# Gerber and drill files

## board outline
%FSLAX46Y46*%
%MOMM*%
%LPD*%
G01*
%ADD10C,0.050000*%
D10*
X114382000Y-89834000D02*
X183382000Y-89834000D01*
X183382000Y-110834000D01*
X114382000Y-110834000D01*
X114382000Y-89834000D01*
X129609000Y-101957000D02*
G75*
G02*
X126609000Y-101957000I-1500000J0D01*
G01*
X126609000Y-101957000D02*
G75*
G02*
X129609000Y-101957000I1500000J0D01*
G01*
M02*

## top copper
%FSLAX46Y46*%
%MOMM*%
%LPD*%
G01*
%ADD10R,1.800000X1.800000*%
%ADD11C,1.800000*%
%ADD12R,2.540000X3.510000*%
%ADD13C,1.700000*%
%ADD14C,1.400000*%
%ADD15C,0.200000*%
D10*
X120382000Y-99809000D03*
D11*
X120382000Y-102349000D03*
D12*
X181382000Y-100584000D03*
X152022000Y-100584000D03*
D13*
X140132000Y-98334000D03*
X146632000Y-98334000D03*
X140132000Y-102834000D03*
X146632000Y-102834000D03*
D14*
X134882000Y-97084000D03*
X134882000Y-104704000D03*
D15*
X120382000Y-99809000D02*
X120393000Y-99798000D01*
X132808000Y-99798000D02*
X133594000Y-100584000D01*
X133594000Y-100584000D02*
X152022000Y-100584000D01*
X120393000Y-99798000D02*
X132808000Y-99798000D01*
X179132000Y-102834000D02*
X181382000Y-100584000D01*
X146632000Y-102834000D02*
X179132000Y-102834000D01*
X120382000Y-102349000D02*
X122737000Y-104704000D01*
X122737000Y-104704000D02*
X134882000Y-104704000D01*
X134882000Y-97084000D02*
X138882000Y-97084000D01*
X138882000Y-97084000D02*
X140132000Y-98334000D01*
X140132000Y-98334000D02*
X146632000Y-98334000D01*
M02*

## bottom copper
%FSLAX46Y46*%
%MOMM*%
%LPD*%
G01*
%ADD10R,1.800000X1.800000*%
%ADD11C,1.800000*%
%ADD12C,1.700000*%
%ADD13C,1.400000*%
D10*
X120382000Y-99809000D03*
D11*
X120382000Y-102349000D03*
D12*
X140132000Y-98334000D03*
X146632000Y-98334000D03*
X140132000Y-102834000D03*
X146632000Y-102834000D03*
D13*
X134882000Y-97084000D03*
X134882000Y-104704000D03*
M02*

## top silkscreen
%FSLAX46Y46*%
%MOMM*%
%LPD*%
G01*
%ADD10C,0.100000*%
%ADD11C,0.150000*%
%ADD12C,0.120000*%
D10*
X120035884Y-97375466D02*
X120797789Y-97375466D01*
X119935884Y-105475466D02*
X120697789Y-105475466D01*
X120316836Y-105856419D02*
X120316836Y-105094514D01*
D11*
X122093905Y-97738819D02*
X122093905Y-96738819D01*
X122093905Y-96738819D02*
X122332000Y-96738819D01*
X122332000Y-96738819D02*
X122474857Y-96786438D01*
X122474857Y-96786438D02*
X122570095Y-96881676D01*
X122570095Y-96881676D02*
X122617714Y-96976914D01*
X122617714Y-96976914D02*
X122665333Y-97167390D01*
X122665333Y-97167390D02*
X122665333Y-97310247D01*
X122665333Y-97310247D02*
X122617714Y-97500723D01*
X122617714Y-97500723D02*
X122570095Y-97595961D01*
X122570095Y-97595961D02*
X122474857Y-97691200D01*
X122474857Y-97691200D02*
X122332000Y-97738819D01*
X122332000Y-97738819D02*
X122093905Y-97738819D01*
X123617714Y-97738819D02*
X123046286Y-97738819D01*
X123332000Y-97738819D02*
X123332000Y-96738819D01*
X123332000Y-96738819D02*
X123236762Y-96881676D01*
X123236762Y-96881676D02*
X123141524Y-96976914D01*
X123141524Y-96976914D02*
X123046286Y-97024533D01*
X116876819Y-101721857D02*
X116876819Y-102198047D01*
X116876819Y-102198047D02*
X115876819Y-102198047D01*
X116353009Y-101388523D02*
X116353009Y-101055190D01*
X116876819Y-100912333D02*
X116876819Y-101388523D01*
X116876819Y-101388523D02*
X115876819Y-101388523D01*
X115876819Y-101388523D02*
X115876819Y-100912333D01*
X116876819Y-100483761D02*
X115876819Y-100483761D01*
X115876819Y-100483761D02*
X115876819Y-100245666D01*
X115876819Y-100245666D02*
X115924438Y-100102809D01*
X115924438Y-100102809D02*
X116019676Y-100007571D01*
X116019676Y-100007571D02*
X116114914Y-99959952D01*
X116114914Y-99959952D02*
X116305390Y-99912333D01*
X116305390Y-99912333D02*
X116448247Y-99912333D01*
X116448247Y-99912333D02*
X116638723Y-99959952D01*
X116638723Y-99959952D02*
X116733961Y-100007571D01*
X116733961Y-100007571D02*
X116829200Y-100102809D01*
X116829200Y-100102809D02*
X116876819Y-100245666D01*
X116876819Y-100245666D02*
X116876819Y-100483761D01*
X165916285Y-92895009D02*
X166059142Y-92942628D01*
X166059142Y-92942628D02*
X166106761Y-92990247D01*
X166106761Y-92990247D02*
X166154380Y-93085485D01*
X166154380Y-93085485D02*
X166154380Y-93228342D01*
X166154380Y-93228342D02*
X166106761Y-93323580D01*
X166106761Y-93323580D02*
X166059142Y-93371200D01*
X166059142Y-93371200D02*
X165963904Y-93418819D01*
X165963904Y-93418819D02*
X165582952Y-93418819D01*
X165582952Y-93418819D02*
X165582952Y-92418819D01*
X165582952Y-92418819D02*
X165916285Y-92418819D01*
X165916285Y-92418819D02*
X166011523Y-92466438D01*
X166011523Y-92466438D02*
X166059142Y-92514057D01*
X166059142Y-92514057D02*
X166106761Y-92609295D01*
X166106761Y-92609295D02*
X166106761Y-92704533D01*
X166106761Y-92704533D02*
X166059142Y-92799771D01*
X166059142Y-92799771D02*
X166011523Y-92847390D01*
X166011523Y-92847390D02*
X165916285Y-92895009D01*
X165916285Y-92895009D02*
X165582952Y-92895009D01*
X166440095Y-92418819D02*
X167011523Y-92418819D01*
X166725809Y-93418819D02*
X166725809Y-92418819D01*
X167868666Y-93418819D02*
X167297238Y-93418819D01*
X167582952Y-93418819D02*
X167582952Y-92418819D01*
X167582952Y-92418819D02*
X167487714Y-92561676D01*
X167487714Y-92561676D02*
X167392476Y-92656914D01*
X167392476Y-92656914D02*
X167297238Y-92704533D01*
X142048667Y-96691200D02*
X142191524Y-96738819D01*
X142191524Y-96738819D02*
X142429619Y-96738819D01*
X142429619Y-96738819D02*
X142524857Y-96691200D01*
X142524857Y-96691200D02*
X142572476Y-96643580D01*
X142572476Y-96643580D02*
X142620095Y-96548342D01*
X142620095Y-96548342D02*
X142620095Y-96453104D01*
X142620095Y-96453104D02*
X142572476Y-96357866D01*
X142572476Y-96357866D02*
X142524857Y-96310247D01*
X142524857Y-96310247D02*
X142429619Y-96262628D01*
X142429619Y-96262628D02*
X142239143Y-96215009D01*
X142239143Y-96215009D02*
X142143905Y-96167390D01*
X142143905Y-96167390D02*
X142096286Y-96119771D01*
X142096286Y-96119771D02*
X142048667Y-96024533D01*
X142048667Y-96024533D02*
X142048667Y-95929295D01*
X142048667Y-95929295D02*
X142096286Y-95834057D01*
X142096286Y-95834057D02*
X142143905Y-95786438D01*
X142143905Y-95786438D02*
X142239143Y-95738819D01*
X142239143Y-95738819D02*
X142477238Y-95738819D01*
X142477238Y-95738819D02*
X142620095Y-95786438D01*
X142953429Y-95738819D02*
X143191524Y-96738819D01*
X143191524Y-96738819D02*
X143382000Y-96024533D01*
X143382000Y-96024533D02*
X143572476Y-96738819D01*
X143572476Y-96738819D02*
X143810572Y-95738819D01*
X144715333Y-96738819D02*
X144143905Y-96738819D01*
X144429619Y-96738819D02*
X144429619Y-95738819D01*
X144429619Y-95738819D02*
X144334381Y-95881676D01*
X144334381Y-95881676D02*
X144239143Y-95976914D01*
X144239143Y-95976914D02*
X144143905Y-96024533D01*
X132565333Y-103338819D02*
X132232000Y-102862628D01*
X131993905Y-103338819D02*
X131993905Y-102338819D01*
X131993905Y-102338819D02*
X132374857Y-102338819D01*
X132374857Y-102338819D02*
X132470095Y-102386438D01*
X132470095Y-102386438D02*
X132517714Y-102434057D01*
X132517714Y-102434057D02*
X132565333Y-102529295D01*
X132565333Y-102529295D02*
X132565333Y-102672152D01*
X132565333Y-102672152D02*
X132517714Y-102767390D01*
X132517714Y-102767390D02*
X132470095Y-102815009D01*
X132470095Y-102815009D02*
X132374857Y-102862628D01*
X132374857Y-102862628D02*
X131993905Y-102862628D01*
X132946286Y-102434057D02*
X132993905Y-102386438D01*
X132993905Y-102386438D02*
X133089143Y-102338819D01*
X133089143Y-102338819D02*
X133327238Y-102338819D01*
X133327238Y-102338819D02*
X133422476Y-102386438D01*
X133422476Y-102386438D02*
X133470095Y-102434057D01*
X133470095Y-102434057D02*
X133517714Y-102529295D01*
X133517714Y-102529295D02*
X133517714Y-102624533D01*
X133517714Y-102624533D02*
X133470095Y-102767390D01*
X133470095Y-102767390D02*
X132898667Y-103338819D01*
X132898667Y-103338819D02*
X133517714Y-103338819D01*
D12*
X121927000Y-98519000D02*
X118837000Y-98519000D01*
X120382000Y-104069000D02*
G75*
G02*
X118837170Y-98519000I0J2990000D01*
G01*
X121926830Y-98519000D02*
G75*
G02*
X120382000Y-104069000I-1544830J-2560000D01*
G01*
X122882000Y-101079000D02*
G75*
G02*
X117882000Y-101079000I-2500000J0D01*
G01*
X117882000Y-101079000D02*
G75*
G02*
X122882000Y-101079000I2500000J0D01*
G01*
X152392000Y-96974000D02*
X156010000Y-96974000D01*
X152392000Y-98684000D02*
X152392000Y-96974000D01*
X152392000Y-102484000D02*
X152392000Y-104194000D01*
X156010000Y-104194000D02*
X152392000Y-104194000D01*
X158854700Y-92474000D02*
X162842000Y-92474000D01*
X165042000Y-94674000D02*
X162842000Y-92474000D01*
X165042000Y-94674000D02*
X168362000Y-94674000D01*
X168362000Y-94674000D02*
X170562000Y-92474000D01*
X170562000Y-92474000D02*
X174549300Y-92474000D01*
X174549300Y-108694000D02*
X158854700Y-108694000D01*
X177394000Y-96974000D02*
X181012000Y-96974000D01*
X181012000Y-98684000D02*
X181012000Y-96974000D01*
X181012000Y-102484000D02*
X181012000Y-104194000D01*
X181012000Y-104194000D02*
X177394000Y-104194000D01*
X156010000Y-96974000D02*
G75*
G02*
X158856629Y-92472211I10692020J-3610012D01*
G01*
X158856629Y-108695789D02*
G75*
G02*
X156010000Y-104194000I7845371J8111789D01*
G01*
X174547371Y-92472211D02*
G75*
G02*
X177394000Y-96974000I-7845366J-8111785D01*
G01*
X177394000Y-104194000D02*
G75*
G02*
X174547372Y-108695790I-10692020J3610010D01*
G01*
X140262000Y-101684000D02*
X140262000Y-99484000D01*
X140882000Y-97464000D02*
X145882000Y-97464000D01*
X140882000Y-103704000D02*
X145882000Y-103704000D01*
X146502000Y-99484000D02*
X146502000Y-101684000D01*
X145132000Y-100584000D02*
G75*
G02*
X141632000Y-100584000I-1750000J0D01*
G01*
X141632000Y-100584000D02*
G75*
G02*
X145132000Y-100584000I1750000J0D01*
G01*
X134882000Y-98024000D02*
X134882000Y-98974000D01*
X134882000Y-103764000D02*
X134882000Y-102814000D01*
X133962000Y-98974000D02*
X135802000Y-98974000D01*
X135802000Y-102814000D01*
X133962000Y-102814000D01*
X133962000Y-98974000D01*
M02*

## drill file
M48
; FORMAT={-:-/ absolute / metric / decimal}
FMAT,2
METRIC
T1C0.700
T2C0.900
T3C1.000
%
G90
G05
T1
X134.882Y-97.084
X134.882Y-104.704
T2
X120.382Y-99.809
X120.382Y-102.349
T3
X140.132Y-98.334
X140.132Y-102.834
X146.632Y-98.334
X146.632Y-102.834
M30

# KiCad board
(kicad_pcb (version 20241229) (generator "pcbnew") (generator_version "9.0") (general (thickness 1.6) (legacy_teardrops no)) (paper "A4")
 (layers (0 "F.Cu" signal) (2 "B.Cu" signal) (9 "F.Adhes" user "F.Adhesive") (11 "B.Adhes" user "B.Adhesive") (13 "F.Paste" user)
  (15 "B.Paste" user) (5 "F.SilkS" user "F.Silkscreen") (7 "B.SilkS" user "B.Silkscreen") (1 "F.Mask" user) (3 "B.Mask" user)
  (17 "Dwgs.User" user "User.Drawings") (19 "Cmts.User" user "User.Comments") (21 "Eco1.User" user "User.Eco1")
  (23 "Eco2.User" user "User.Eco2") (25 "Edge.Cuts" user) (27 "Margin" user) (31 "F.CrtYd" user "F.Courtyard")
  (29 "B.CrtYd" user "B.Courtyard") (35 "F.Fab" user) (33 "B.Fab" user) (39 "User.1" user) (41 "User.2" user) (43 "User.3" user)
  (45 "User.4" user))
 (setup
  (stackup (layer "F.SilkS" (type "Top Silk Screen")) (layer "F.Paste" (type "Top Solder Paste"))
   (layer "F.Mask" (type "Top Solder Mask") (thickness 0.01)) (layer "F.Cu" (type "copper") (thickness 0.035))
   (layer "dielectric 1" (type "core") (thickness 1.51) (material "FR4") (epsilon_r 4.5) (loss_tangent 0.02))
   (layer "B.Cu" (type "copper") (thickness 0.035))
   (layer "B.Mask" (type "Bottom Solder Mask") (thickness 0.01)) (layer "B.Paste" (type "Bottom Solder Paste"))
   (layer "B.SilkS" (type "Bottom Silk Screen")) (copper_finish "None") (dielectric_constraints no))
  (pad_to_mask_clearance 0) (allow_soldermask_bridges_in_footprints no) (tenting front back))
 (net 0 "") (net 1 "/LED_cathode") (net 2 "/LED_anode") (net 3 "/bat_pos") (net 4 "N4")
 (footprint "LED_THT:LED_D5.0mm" (layer "F.Cu") (at 120.382 99.809 -90)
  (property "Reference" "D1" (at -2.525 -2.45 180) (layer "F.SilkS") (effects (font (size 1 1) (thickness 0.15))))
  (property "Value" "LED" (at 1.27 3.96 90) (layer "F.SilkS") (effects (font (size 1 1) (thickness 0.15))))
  (fp_line (start -1.29 -1.545) (end -1.29 1.545) (stroke (width 0.12) (type solid)) (layer "F.SilkS"))
  (fp_arc (start 4.26 0) (mid 2.071779 2.880495) (end -1.29 1.54483) (stroke (width 0.12) (type solid)) (layer "F.SilkS"))
  (fp_arc (start -1.29 -1.54483) (mid 2.071779 -2.880495) (end 4.26 0) (stroke (width 0.12) (type solid)) (layer "F.SilkS"))
  (fp_circle (center 1.27 0) (end 3.77 0) (stroke (width 0.12) (type solid)) (fill no) (layer "F.SilkS"))
  (pad "1" thru_hole rect (at 0 0 270) (size 1.8 1.8) (drill 0.9) (layers "*.Cu" "*.Mask") (remove_unused_layers no) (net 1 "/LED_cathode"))
  (pad "2" thru_hole circle (at 2.54 0 270) (size 1.8 1.8) (drill 0.9) (layers "*.Cu" "*.Mask") (remove_unused_layers no)
   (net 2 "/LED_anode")))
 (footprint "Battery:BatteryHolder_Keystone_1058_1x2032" (layer "F.Cu") (at 166.702 100.584 180)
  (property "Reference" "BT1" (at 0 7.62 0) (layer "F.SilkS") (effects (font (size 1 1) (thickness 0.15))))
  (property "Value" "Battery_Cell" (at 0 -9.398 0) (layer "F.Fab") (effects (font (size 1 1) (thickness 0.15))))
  (fp_line (start 14.31 3.61) (end 10.692 3.61) (stroke (width 0.12) (type solid)) (layer "F.SilkS"))
  (fp_line (start 14.31 1.9) (end 14.31 3.61) (stroke (width 0.12) (type solid)) (layer "F.SilkS"))
  (fp_line (start 14.31 -1.9) (end 14.31 -3.61) (stroke (width 0.12) (type solid)) (layer "F.SilkS"))
  (fp_line (start 10.692 -3.61) (end 14.31 -3.61) (stroke (width 0.12) (type solid)) (layer "F.SilkS"))
  (fp_line (start 7.8473 8.11) (end 3.86 8.11) (stroke (width 0.12) (type solid)) (layer "F.SilkS"))
  (fp_line (start 1.66 5.91) (end 3.86 8.11) (stroke (width 0.12) (type solid)) (layer "F.SilkS"))
  (fp_line (start 1.66 5.91) (end -1.66 5.91) (stroke (width 0.12) (type solid)) (layer "F.SilkS"))
  (fp_line (start -1.66 5.91) (end -3.86 8.11) (stroke (width 0.12) (type solid)) (layer "F.SilkS"))
  (fp_line (start -3.86 8.11) (end -7.8473 8.11) (stroke (width 0.12) (type solid)) (layer "F.SilkS"))
  (fp_line (start -7.8473 -8.11) (end 7.8473 -8.11) (stroke (width 0.12) (type solid)) (layer "F.SilkS"))
  (fp_line (start -10.692 3.61) (end -14.31 3.61) (stroke (width 0.12) (type solid)) (layer "F.SilkS"))
  (fp_line (start -14.31 1.9) (end -14.31 3.61) (stroke (width 0.12) (type solid)) (layer "F.SilkS"))
  (fp_line (start -14.31 -1.9) (end -14.31 -3.61) (stroke (width 0.12) (type solid)) (layer "F.SilkS"))
  (fp_line (start -14.31 -3.61) (end -10.692 -3.61) (stroke (width 0.12) (type solid)) (layer "F.SilkS"))
  (fp_arc (start 10.692 3.61) (mid 9.538084 6.031244) (end 7.845371 8.111789) (stroke (width 0.12) (type solid)) (layer "F.SilkS"))
  (fp_arc (start 7.845371 -8.111789) (mid 9.538085 -6.031244) (end 10.692 -3.61) (stroke (width 0.12) (type solid)) (layer "F.SilkS"))
  (fp_arc (start -7.845371 8.111789) (mid -9.538085 6.031244) (end -10.692 3.61) (stroke (width 0.12) (type solid)) (layer "F.SilkS"))
  (fp_arc (start -10.692 -3.61) (mid -9.538084 -6.031244) (end -7.845371 -8.111789) (stroke (width 0.12) (type solid)) (layer "F.SilkS"))
  (pad "1" smd rect (at -14.68 0 180) (size 2.54 3.51) (layers "F.Cu" "F.Mask" "F.Paste") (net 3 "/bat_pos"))
  (pad "2" smd rect (at 14.68 0 180) (size 2.54 3.51) (layers "F.Cu" "F.Mask" "F.Paste") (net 1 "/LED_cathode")))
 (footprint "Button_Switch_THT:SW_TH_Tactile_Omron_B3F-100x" (layer "F.Cu") (at 140.132 98.334)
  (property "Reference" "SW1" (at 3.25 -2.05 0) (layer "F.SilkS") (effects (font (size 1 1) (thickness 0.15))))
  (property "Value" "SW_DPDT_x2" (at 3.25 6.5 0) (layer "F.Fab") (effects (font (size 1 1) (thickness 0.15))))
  (fp_line (start 0.13 3.35) (end 0.13 1.15) (stroke (width 0.12) (type solid)) (layer "F.SilkS"))
  (fp_line (start 0.75 -0.87) (end 5.75 -0.87) (stroke (width 0.12) (type solid)) (layer "F.SilkS"))
  (fp_line (start 0.75 5.37) (end 5.75 5.37) (stroke (width 0.12) (type solid)) (layer "F.SilkS"))
  (fp_line (start 6.37 1.15) (end 6.37 3.35) (stroke (width 0.12) (type solid)) (layer "F.SilkS"))
  (fp_circle (center 3.25 2.25) (end 5 2.25) (stroke (width 0.12) (type solid)) (fill no) (layer "F.SilkS"))
  (pad "1" thru_hole circle (at 0 0) (size 1.7 1.7) (drill 1) (layers "*.Cu" "*.Mask") (remove_unused_layers no) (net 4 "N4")
   (thermal_bridge_angle 90))
  (pad "1" thru_hole circle (at 6.5 0) (size 1.7 1.7) (drill 1) (layers "*.Cu" "*.Mask") (remove_unused_layers no) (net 4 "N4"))
  (pad "2" thru_hole circle (at 0 4.5) (size 1.7 1.7) (drill 1) (layers "*.Cu" "*.Mask") (remove_unused_layers no) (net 3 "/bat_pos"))
  (pad "2" thru_hole circle (at 6.5 4.5) (size 1.7 1.7) (drill 1) (layers "*.Cu" "*.Mask") (remove_unused_layers no) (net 3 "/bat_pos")))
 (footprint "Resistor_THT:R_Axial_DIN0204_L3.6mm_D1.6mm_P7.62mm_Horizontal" (layer "F.Cu") (at 134.882 97.084 -90)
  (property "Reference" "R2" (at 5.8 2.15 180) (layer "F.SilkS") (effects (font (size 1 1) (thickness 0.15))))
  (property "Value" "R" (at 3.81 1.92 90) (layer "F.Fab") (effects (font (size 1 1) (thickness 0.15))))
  (fp_line (start 0.94 0) (end 1.89 0) (stroke (width 0.12) (type solid)) (layer "F.SilkS"))
  (fp_line (start 6.68 0) (end 5.73 0) (stroke (width 0.12) (type solid)) (layer "F.SilkS"))
  (fp_rect (start 1.89 -0.92) (end 5.73 0.92) (stroke (width 0.12) (type solid)) (fill no) (layer "F.SilkS"))
  (pad "1" thru_hole circle (at 0 0 270) (size 1.4 1.4) (drill 0.7) (layers "*.Cu" "*.Mask") (remove_unused_layers no) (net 4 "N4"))
  (pad "2" thru_hole circle (at 7.62 0 270) (size 1.4 1.4) (drill 0.7) (layers "*.Cu" "*.Mask") (remove_unused_layers no)
   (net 2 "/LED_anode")))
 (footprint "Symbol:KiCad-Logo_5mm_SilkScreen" (layer "B.Cu") (at 167.132 100.584 180)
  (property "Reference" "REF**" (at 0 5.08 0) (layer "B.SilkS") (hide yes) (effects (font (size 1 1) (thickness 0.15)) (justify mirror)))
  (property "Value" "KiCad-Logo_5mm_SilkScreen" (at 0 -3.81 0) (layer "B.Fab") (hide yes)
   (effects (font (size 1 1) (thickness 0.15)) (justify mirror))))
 (gr_rect (start 114.382 89.834) (end 183.382 110.834) (stroke (width 0.05) (type default)) (fill no) (layer "Edge.Cuts"))
 (gr_circle (center 128.109 101.957) (end 128.109 100.457) (stroke (width 0.05) (type default)) (fill no) (layer "Edge.Cuts"))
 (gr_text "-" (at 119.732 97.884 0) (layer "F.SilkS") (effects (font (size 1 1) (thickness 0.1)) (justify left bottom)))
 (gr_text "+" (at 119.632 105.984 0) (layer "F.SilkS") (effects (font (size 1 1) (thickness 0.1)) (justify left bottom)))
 (segment (start 120.382 99.809) (end 120.393 99.798) (width 0.2) (layer "F.Cu") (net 1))
 (segment (start 132.808 99.798) (end 133.594 100.584) (width 0.2) (layer "F.Cu") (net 1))
 (segment (start 133.594 100.584) (end 152.022 100.584) (width 0.2) (layer "F.Cu") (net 1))
 (segment (start 120.393 99.798) (end 132.808 99.798) (width 0.2) (layer "F.Cu") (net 1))
 (segment (start 179.132 102.834) (end 181.382 100.584) (width 0.2) (layer "F.Cu") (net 3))
 (segment (start 146.632 102.834) (end 179.132 102.834) (width 0.2) (layer "F.Cu") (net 3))
 (segment (start 120.382 102.349) (end 122.737 104.704) (width 0.2) (layer "F.Cu") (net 2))
 (segment (start 122.737 104.704) (end 134.882 104.704) (width 0.2) (layer "F.Cu") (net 2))
 (segment (start 134.882 97.084) (end 138.882 97.084) (width 0.2) (layer "F.Cu") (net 4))
 (segment (start 138.882 97.084) (end 140.132 98.334) (width 0.2) (layer "F.Cu") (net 4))
 (segment (start 140.132 98.334) (end 146.632 98.334) (width 0.2) (layer "F.Cu") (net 4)))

